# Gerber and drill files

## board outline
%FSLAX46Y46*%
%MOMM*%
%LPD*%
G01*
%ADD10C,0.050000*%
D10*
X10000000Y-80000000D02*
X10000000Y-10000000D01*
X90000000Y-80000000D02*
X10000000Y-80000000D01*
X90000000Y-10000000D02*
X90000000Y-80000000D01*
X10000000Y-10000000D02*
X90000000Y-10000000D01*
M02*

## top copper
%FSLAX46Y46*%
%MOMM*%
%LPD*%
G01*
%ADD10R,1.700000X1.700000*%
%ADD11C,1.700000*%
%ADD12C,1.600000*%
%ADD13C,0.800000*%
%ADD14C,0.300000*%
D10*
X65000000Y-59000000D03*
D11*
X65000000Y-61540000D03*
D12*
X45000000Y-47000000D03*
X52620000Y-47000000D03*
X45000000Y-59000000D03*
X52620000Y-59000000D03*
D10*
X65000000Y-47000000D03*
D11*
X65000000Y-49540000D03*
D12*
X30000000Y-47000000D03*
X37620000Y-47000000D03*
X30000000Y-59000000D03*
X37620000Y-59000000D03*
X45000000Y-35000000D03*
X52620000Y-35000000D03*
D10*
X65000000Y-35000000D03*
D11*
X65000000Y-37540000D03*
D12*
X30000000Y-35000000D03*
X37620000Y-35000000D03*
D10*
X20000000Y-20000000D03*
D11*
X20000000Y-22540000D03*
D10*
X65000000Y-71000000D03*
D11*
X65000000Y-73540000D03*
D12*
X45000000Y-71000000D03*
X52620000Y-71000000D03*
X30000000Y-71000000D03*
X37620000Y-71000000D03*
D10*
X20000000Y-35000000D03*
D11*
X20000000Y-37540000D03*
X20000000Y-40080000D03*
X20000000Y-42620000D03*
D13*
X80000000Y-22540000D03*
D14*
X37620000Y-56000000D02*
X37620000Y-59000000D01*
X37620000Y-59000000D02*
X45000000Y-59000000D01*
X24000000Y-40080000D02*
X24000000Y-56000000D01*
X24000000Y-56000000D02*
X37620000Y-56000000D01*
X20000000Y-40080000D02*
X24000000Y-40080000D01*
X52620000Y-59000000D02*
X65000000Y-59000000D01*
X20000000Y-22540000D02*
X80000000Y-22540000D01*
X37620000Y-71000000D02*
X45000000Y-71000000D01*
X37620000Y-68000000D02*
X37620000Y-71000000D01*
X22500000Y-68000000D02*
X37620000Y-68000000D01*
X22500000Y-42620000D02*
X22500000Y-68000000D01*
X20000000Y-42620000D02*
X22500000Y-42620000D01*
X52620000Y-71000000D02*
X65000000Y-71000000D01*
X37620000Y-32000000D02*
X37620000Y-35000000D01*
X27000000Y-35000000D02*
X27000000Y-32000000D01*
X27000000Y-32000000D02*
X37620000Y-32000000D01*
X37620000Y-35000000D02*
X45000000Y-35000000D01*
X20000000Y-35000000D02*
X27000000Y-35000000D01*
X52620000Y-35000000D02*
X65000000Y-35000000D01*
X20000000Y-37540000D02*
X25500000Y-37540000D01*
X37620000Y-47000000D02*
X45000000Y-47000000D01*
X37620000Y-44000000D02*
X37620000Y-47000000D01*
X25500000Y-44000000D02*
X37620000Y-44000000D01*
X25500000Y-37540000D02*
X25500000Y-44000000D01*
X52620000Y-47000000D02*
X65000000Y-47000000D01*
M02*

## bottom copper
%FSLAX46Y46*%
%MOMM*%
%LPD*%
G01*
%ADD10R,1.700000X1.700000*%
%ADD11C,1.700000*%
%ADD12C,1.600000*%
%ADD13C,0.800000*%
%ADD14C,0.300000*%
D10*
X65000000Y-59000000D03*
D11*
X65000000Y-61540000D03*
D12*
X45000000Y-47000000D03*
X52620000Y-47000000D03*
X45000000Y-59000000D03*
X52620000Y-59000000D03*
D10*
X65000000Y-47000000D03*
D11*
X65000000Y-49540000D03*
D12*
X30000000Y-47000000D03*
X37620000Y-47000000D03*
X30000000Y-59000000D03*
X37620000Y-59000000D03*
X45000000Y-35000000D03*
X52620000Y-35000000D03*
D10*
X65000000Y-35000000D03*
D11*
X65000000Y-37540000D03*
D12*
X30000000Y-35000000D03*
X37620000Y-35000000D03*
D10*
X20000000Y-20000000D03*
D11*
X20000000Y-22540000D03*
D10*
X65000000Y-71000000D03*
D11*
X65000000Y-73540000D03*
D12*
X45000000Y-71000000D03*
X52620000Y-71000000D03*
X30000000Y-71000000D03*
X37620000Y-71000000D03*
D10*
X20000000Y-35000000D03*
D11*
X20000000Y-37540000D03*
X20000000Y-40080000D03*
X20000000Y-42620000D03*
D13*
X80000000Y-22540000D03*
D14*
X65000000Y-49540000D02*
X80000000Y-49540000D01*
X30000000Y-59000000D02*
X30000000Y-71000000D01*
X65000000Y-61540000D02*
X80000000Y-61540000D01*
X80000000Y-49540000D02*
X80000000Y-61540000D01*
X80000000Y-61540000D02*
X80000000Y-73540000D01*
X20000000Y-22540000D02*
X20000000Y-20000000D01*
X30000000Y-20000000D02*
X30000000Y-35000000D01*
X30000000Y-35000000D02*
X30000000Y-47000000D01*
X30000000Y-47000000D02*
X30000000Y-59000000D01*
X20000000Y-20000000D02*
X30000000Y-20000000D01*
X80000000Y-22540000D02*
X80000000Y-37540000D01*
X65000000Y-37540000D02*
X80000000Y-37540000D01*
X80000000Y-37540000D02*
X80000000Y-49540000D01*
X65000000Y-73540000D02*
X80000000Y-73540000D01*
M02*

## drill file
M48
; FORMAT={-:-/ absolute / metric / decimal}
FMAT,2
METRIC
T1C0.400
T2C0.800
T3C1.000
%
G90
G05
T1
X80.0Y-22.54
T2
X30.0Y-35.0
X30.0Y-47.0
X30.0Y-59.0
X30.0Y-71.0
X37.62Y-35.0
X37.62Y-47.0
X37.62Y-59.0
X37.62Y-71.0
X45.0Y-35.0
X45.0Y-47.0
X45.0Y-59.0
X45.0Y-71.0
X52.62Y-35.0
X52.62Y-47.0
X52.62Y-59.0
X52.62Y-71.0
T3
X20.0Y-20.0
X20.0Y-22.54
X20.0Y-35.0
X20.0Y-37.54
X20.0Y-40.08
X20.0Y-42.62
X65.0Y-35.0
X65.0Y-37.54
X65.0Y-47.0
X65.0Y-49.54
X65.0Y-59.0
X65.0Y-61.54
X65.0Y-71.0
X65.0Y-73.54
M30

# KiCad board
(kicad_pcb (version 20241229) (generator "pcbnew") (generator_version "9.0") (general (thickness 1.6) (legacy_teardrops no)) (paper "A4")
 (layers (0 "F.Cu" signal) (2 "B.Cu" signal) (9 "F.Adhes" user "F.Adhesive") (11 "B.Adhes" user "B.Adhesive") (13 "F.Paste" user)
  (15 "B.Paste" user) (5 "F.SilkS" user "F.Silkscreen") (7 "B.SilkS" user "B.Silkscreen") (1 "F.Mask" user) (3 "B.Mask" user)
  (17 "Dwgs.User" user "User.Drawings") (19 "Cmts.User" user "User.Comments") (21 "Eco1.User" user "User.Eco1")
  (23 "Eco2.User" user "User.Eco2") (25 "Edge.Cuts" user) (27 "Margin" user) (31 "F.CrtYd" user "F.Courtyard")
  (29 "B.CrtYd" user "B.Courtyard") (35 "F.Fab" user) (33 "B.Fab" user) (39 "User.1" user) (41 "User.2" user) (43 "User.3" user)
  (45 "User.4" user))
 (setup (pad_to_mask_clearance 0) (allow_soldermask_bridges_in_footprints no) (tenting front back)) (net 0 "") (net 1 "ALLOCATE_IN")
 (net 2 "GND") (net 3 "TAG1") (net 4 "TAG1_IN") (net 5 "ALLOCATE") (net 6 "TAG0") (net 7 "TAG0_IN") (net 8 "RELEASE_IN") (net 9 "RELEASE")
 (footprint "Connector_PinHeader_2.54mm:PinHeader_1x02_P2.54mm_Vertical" (layer "F.Cu") (at 65 59)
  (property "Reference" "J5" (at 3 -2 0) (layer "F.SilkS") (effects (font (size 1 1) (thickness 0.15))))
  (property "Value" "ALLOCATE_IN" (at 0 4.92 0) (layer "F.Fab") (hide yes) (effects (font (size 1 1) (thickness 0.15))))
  (pad "1" thru_hole rect (at 0 0) (size 1.7 1.7) (drill 1) (layers "*.Cu" "*.Mask") (remove_unused_layers no) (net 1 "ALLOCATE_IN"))
  (pad "2" thru_hole circle (at 0 2.54) (size 1.7 1.7) (drill 1) (layers "*.Cu" "*.Mask") (remove_unused_layers no) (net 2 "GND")))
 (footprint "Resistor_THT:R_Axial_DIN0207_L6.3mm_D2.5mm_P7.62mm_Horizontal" (layer "F.Cu") (at 45 47)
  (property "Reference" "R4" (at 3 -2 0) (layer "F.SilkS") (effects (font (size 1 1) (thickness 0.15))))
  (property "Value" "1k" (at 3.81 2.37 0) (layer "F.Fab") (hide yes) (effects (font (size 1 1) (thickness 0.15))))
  (pad "1" thru_hole circle (at 0 0) (size 1.6 1.6) (drill 0.8) (layers "*.Cu" "*.Mask") (remove_unused_layers no) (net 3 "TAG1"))
  (pad "2" thru_hole circle (at 7.62 0) (size 1.6 1.6) (drill 0.8) (layers "*.Cu" "*.Mask") (remove_unused_layers no) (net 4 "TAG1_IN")))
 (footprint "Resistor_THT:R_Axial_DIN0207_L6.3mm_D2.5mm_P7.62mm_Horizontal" (layer "F.Cu") (at 45 59)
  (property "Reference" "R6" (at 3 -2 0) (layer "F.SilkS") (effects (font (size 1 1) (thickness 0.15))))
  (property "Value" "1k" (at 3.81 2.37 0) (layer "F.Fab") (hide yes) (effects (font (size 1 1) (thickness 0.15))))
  (pad "1" thru_hole circle (at 0 0) (size 1.6 1.6) (drill 0.8) (layers "*.Cu" "*.Mask") (remove_unused_layers no) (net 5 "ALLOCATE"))
  (pad "2" thru_hole circle (at 7.62 0) (size 1.6 1.6) (drill 0.8) (layers "*.Cu" "*.Mask") (remove_unused_layers no) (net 1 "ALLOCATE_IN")))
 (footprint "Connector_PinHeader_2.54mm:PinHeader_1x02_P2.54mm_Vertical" (layer "F.Cu") (at 65 47)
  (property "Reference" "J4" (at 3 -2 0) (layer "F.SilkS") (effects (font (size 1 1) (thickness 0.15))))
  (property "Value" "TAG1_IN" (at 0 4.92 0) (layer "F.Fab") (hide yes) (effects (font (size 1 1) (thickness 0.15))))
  (pad "1" thru_hole rect (at 0 0) (size 1.7 1.7) (drill 1) (layers "*.Cu" "*.Mask") (remove_unused_layers no) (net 4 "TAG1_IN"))
  (pad "2" thru_hole circle (at 0 2.54) (size 1.7 1.7) (drill 1) (layers "*.Cu" "*.Mask") (remove_unused_layers no) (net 2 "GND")))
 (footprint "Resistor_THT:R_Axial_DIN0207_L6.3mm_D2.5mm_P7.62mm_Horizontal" (layer "F.Cu") (at 30 47)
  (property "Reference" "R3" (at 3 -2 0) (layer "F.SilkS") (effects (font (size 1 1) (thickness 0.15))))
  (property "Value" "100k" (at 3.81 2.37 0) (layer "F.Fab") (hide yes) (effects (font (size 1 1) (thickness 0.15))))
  (pad "1" thru_hole circle (at 0 0) (size 1.6 1.6) (drill 0.8) (layers "*.Cu" "*.Mask") (remove_unused_layers no) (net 2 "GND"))
  (pad "2" thru_hole circle (at 7.62 0) (size 1.6 1.6) (drill 0.8) (layers "*.Cu" "*.Mask") (remove_unused_layers no) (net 3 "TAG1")))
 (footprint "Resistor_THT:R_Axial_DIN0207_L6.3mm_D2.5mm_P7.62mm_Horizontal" (layer "F.Cu") (at 30 59)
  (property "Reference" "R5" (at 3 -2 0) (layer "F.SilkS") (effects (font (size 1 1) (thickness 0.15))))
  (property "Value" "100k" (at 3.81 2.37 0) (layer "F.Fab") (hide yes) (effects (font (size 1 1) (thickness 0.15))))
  (pad "1" thru_hole circle (at 0 0) (size 1.6 1.6) (drill 0.8) (layers "*.Cu" "*.Mask") (remove_unused_layers no) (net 2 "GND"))
  (pad "2" thru_hole circle (at 7.62 0) (size 1.6 1.6) (drill 0.8) (layers "*.Cu" "*.Mask") (remove_unused_layers no) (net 5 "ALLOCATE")))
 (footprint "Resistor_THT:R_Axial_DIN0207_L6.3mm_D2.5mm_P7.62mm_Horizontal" (layer "F.Cu") (at 45 35)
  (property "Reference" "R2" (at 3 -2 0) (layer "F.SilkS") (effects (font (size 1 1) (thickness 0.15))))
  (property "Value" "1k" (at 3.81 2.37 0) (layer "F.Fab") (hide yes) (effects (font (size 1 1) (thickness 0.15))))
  (pad "1" thru_hole circle (at 0 0) (size 1.6 1.6) (drill 0.8) (layers "*.Cu" "*.Mask") (remove_unused_layers no) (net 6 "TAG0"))
  (pad "2" thru_hole circle (at 7.62 0) (size 1.6 1.6) (drill 0.8) (layers "*.Cu" "*.Mask") (remove_unused_layers no) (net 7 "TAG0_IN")))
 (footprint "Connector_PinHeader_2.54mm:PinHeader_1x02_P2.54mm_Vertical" (layer "F.Cu") (at 65 35)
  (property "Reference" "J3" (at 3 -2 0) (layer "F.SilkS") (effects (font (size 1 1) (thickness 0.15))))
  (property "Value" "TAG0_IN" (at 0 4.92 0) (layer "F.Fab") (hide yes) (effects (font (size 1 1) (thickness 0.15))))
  (pad "1" thru_hole rect (at 0 0) (size 1.7 1.7) (drill 1) (layers "*.Cu" "*.Mask") (remove_unused_layers no) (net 7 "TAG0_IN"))
  (pad "2" thru_hole circle (at 0 2.54) (size 1.7 1.7) (drill 1) (layers "*.Cu" "*.Mask") (remove_unused_layers no) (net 2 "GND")))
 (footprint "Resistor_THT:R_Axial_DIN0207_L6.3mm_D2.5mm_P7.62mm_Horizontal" (layer "F.Cu") (at 30 35)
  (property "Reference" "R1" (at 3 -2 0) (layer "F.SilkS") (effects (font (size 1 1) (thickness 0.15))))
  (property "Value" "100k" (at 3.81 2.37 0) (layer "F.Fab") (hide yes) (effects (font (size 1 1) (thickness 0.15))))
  (pad "1" thru_hole circle (at 0 0) (size 1.6 1.6) (drill 0.8) (layers "*.Cu" "*.Mask") (remove_unused_layers no) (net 2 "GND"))
  (pad "2" thru_hole circle (at 7.62 0) (size 1.6 1.6) (drill 0.8) (layers "*.Cu" "*.Mask") (remove_unused_layers no) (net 6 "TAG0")))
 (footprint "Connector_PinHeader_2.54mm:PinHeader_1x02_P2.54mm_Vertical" (layer "F.Cu") (at 20 20)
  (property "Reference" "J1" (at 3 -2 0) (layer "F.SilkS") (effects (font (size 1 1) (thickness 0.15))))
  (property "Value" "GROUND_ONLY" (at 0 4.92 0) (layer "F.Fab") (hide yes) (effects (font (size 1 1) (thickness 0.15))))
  (pad "1" thru_hole rect (at 0 0) (size 1.7 1.7) (drill 1) (layers "*.Cu" "*.Mask") (remove_unused_layers no) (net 2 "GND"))
  (pad "2" thru_hole circle (at 0 2.54) (size 1.7 1.7) (drill 1) (layers "*.Cu" "*.Mask") (remove_unused_layers no) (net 2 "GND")))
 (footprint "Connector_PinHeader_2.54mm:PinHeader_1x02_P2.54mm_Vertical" (layer "F.Cu") (at 65 71)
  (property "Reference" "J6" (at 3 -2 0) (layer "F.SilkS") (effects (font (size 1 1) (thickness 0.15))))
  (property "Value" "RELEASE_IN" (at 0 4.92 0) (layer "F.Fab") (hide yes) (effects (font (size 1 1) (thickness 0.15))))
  (pad "1" thru_hole rect (at 0 0) (size 1.7 1.7) (drill 1) (layers "*.Cu" "*.Mask") (remove_unused_layers no) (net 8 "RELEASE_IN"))
  (pad "2" thru_hole circle (at 0 2.54) (size 1.7 1.7) (drill 1) (layers "*.Cu" "*.Mask") (remove_unused_layers no) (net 2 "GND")))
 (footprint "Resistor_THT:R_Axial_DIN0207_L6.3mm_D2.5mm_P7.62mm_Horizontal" (layer "F.Cu") (at 45 71)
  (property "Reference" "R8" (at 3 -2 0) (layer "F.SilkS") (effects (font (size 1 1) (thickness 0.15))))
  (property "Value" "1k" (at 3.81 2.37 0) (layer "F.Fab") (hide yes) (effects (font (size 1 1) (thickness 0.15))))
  (pad "1" thru_hole circle (at 0 0) (size 1.6 1.6) (drill 0.8) (layers "*.Cu" "*.Mask") (remove_unused_layers no) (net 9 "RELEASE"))
  (pad "2" thru_hole circle (at 7.62 0) (size 1.6 1.6) (drill 0.8) (layers "*.Cu" "*.Mask") (remove_unused_layers no) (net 8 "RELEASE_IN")))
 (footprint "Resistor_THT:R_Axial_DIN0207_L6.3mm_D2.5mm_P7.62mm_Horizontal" (layer "F.Cu") (at 30 71)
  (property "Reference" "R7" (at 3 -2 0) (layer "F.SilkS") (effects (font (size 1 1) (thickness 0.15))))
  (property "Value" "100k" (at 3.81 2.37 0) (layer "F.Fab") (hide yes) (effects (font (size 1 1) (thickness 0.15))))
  (pad "1" thru_hole circle (at 0 0) (size 1.6 1.6) (drill 0.8) (layers "*.Cu" "*.Mask") (remove_unused_layers no) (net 2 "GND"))
  (pad "2" thru_hole circle (at 7.62 0) (size 1.6 1.6) (drill 0.8) (layers "*.Cu" "*.Mask") (remove_unused_layers no) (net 9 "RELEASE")))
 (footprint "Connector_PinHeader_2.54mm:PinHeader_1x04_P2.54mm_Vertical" (layer "F.Cu") (at 20 35)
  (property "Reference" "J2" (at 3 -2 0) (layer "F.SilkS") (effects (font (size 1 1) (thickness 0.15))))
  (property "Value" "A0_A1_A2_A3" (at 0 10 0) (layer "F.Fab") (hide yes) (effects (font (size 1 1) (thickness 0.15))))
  (pad "1" thru_hole rect (at 0 0) (size 1.7 1.7) (drill 1) (layers "*.Cu" "*.Mask") (remove_unused_layers no) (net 6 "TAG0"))
  (pad "2" thru_hole circle (at 0 2.54) (size 1.7 1.7) (drill 1) (layers "*.Cu" "*.Mask") (remove_unused_layers no) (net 3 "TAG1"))
  (pad "3" thru_hole circle (at 0 5.08) (size 1.7 1.7) (drill 1) (layers "*.Cu" "*.Mask") (remove_unused_layers no) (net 5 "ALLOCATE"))
  (pad "4" thru_hole circle (at 0 7.62) (size 1.7 1.7) (drill 1) (layers "*.Cu" "*.Mask") (remove_unused_layers no) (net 9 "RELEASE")))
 (gr_line (start 10 80) (end 10 10) (stroke (width 0.05) (type default)) (layer "Edge.Cuts"))
 (gr_line (start 90 80) (end 10 80) (stroke (width 0.05) (type default)) (layer "Edge.Cuts"))
 (gr_line (start 90 10) (end 90 80) (stroke (width 0.05) (type default)) (layer "Edge.Cuts"))
 (gr_line (start 10 10) (end 90 10) (stroke (width 0.05) (type default)) (layer "Edge.Cuts"))
 (segment (start 37.62 56) (end 37.62 59) (width 0.3) (layer "F.Cu") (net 5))
 (segment (start 37.62 59) (end 45 59) (width 0.3) (layer "F.Cu") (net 5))
 (segment (start 24 40.08) (end 24 56) (width 0.3) (layer "F.Cu") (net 5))
 (segment (start 24 56) (end 37.62 56) (width 0.3) (layer "F.Cu") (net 5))
 (segment (start 20 40.08) (end 24 40.08) (width 0.3) (layer "F.Cu") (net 5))
 (segment (start 52.62 59) (end 65 59) (width 0.3) (layer "F.Cu") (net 1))
 (segment (start 20 22.54) (end 80 22.54) (width 0.3) (layer "F.Cu") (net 2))
 (via (at 80 22.54) (size 0.8) (drill 0.4) (layers "F.Cu" "B.Cu") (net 2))
 (segment (start 65 49.54) (end 80 49.54) (width 0.3) (layer "B.Cu") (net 2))
 (segment (start 30 59) (end 30 71) (width 0.3) (layer "B.Cu") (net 2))
 (segment (start 65 61.54) (end 80 61.54) (width 0.3) (layer "B.Cu") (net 2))
 (segment (start 80 49.54) (end 80 61.54) (width 0.3) (layer "B.Cu") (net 2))
 (segment (start 80 61.54) (end 80 73.54) (width 0.3) (layer "B.Cu") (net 2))
 (segment (start 20 22.54) (end 20 20) (width 0.3) (layer "B.Cu") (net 2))
 (segment (start 30 20) (end 30 35) (width 0.3) (layer "B.Cu") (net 2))
 (segment (start 30 35) (end 30 47) (width 0.3) (layer "B.Cu") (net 2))
 (segment (start 30 47) (end 30 59) (width 0.3) (layer "B.Cu") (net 2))
 (segment (start 20 20) (end 30 20) (width 0.3) (layer "B.Cu") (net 2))
 (segment (start 80 22.54) (end 80 37.54) (width 0.3) (layer "B.Cu") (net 2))
 (segment (start 65 37.54) (end 80 37.54) (width 0.3) (layer "B.Cu") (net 2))
 (segment (start 80 37.54) (end 80 49.54) (width 0.3) (layer "B.Cu") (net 2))
 (segment (start 65 73.54) (end 80 73.54) (width 0.3) (layer "B.Cu") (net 2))
 (segment (start 37.62 71) (end 45 71) (width 0.3) (layer "F.Cu") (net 9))
 (segment (start 37.62 68) (end 37.62 71) (width 0.3) (layer "F.Cu") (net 9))
 (segment (start 22.5 68) (end 37.62 68) (width 0.3) (layer "F.Cu") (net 9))
 (segment (start 22.5 42.62) (end 22.5 68) (width 0.3) (layer "F.Cu") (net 9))
 (segment (start 20 42.62) (end 22.5 42.62) (width 0.3) (layer "F.Cu") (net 9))
 (segment (start 52.62 71) (end 65 71) (width 0.3) (layer "F.Cu") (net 8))
 (segment (start 37.62 32) (end 37.62 35) (width 0.3) (layer "F.Cu") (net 6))
 (segment (start 27 35) (end 27 32) (width 0.3) (layer "F.Cu") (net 6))
 (segment (start 27 32) (end 37.62 32) (width 0.3) (layer "F.Cu") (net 6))
 (segment (start 37.62 35) (end 45 35) (width 0.3) (layer "F.Cu") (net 6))
 (segment (start 20 35) (end 27 35) (width 0.3) (layer "F.Cu") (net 6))
 (segment (start 52.62 35) (end 65 35) (width 0.3) (layer "F.Cu") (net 7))
 (segment (start 20 37.54) (end 25.5 37.54) (width 0.3) (layer "F.Cu") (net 3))
 (segment (start 37.62 47) (end 45 47) (width 0.3) (layer "F.Cu") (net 3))
 (segment (start 37.62 44) (end 37.62 47) (width 0.3) (layer "F.Cu") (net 3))
 (segment (start 25.5 44) (end 37.62 44) (width 0.3) (layer "F.Cu") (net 3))
 (segment (start 25.5 37.54) (end 25.5 44) (width 0.3) (layer "F.Cu") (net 3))
 (segment (start 52.62 47) (end 65 47) (width 0.3) (layer "F.Cu") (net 4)))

